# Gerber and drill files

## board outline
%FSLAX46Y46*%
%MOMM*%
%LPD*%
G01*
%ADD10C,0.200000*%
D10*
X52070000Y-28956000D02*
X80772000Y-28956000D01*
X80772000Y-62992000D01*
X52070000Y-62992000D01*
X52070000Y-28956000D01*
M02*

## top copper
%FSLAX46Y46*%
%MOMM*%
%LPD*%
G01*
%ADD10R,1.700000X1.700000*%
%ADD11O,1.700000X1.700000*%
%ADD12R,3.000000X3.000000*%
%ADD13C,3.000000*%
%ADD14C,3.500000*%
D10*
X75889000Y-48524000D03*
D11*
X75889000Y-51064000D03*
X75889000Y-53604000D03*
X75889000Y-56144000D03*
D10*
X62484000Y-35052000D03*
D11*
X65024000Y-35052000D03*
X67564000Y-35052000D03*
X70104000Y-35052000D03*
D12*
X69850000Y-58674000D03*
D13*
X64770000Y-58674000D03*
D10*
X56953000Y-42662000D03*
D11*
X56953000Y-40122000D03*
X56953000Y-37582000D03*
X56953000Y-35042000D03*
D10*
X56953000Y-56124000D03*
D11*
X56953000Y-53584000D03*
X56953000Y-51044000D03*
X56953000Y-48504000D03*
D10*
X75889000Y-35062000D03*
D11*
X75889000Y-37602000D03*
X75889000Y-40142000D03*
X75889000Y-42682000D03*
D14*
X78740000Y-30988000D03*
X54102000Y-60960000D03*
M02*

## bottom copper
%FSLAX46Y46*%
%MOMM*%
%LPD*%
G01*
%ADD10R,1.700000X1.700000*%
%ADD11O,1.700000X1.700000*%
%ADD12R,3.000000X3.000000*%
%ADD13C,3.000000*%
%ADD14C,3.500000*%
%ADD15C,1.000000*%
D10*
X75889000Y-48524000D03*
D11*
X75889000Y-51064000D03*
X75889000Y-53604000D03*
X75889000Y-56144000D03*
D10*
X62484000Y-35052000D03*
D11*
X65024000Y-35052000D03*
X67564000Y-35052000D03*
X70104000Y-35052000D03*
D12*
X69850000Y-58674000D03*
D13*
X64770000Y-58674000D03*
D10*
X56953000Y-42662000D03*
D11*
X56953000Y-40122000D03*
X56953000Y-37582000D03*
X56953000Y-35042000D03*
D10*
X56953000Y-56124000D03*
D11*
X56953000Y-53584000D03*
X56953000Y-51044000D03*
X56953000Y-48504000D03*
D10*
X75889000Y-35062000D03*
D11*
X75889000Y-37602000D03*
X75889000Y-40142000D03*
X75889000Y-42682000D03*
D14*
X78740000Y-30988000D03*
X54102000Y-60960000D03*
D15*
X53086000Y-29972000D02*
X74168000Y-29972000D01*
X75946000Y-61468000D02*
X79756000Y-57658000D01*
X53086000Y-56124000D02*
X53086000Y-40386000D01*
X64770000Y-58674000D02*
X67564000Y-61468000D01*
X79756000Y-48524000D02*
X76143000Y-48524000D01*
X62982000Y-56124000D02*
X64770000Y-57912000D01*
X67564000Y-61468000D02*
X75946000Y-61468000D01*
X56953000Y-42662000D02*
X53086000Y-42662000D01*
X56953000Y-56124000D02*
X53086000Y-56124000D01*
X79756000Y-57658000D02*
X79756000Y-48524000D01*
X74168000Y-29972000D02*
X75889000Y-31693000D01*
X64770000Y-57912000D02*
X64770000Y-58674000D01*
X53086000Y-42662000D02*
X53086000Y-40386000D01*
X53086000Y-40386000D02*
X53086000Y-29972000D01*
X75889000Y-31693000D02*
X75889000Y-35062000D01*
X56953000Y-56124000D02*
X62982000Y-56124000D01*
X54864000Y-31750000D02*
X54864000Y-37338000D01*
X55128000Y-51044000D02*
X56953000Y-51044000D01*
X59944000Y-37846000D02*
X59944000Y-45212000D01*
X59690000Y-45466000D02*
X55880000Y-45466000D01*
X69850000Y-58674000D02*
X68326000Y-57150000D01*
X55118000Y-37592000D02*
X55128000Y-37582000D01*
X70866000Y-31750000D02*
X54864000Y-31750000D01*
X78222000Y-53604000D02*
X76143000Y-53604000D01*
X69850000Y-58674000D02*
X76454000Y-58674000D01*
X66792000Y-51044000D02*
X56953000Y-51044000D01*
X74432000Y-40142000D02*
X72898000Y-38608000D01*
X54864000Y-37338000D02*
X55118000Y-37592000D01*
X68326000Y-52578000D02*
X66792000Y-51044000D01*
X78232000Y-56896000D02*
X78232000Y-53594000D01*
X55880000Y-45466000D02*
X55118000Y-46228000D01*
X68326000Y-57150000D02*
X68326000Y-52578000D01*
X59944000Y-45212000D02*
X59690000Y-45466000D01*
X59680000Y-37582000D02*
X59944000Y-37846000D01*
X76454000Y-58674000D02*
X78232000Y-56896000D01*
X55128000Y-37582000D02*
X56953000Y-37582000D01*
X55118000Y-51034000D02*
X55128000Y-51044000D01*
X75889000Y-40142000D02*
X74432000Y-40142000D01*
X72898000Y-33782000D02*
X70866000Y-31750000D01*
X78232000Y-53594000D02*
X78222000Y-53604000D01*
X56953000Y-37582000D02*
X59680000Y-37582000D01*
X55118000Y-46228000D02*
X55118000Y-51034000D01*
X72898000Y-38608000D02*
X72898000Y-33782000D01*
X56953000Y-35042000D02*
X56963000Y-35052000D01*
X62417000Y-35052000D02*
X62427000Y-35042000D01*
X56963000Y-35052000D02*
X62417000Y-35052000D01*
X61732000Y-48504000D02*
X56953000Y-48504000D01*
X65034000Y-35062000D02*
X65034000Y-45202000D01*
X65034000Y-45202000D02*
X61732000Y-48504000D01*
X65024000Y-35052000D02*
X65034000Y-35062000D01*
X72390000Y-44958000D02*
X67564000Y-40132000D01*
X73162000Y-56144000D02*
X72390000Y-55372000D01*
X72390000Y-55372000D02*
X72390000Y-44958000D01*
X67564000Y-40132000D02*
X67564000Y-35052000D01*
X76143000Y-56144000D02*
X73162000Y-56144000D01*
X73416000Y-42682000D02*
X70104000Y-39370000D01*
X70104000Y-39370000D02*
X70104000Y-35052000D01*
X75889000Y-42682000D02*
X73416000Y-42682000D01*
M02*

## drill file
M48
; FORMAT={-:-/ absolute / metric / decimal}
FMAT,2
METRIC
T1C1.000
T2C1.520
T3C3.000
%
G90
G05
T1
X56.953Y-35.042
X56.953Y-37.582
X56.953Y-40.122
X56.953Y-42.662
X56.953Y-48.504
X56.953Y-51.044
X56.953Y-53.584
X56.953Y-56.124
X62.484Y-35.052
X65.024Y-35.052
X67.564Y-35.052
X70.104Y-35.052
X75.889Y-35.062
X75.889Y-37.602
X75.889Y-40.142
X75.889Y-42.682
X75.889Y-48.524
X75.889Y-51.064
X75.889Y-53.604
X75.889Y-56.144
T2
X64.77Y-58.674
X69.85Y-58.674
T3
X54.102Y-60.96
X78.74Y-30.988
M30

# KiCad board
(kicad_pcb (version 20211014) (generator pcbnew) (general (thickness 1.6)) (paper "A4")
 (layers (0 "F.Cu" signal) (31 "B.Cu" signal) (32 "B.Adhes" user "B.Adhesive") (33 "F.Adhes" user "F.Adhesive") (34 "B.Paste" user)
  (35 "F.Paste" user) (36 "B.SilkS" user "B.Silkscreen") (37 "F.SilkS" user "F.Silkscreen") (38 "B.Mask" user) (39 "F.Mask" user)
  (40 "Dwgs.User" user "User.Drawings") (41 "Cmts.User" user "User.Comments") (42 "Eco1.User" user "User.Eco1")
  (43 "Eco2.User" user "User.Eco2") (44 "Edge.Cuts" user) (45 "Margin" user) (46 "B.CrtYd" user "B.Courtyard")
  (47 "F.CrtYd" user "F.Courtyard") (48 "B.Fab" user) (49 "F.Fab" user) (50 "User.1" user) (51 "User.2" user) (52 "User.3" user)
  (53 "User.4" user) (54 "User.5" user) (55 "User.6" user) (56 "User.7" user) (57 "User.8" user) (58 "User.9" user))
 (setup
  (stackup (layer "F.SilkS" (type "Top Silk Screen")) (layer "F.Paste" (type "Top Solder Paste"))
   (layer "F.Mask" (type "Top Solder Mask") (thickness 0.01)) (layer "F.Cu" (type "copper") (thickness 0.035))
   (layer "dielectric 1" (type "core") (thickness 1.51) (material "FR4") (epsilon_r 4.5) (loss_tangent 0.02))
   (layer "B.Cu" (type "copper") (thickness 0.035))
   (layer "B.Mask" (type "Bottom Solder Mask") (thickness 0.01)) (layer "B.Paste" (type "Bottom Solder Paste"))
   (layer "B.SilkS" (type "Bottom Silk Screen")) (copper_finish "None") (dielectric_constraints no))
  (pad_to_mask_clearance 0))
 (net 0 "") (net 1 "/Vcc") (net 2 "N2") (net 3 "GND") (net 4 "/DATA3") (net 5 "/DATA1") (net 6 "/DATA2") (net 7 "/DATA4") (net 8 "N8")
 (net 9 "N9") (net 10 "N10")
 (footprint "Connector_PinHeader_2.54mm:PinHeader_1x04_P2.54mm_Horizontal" (layer "F.Cu") (at 75.889 48.524)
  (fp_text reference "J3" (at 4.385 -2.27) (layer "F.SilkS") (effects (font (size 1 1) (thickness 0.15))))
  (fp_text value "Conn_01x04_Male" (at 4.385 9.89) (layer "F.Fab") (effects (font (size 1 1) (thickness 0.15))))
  (pad "1" thru_hole rect (at 0 0) (size 1.7 1.7) (drill 1) (layers *.Cu *.Mask) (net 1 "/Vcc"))
  (pad "2" thru_hole oval (at 0 2.54) (size 1.7 1.7) (drill 1) (layers *.Cu *.Mask) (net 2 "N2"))
  (pad "3" thru_hole oval (at 0 5.08) (size 1.7 1.7) (drill 1) (layers *.Cu *.Mask) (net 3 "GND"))
  (pad "4" thru_hole oval (at 0 7.62) (size 1.7 1.7) (drill 1) (layers *.Cu *.Mask) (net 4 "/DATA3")))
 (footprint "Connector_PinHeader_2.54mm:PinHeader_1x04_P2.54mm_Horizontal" (layer "F.Cu") (at 62.484 35.052 90)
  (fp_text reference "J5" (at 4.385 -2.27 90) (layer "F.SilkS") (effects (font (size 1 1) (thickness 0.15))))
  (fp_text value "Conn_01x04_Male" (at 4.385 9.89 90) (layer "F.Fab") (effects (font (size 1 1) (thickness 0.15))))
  (pad "1" thru_hole rect (at 0 0 90) (size 1.7 1.7) (drill 1) (layers *.Cu *.Mask) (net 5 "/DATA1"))
  (pad "2" thru_hole oval (at 0 2.54 90) (size 1.7 1.7) (drill 1) (layers *.Cu *.Mask) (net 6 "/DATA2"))
  (pad "3" thru_hole oval (at 0 5.08 90) (size 1.7 1.7) (drill 1) (layers *.Cu *.Mask) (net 4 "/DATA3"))
  (pad "4" thru_hole oval (at 0 7.62 90) (size 1.7 1.7) (drill 1) (layers *.Cu *.Mask) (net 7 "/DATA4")))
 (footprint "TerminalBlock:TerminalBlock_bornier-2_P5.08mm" (layer "F.Cu") (at 69.85 58.674 180)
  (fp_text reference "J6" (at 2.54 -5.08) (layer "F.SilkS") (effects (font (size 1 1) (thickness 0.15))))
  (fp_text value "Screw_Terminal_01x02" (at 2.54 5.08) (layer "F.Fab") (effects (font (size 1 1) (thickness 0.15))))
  (pad "1" thru_hole rect (at 0 0 180) (size 3 3) (drill 1.52) (layers *.Cu *.Mask) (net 3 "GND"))
  (pad "2" thru_hole circle (at 5.08 0 180) (size 3 3) (drill 1.52) (layers *.Cu *.Mask) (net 1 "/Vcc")))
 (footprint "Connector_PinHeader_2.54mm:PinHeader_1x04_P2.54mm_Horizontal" (layer "F.Cu") (at 56.953 42.662 180)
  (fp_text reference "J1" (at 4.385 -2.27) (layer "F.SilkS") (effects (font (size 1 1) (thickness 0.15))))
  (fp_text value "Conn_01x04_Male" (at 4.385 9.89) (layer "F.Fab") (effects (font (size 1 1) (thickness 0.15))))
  (pad "1" thru_hole rect (at 0 0 180) (size 1.7 1.7) (drill 1) (layers *.Cu *.Mask) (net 1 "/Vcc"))
  (pad "2" thru_hole oval (at 0 2.54 180) (size 1.7 1.7) (drill 1) (layers *.Cu *.Mask) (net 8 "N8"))
  (pad "3" thru_hole oval (at 0 5.08 180) (size 1.7 1.7) (drill 1) (layers *.Cu *.Mask) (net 3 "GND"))
  (pad "4" thru_hole oval (at 0 7.62 180) (size 1.7 1.7) (drill 1) (layers *.Cu *.Mask) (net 5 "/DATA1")))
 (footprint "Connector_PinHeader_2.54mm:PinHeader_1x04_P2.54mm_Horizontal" (layer "F.Cu") (at 56.953 56.124 180)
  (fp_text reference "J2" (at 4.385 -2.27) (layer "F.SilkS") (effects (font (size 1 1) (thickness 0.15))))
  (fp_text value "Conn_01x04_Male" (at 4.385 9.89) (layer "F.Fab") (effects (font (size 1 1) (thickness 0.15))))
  (pad "1" thru_hole rect (at 0 0 180) (size 1.7 1.7) (drill 1) (layers *.Cu *.Mask) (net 1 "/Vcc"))
  (pad "2" thru_hole oval (at 0 2.54 180) (size 1.7 1.7) (drill 1) (layers *.Cu *.Mask) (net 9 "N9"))
  (pad "3" thru_hole oval (at 0 5.08 180) (size 1.7 1.7) (drill 1) (layers *.Cu *.Mask) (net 3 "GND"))
  (pad "4" thru_hole oval (at 0 7.62 180) (size 1.7 1.7) (drill 1) (layers *.Cu *.Mask) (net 6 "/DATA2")))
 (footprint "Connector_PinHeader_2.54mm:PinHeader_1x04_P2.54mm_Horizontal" (layer "F.Cu") (at 75.889 35.062)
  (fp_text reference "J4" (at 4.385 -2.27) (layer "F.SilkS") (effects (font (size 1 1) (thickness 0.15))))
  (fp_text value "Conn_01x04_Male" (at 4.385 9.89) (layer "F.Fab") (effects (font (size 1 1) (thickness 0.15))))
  (pad "1" thru_hole rect (at 0 0) (size 1.7 1.7) (drill 1) (layers *.Cu *.Mask) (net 1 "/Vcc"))
  (pad "2" thru_hole oval (at 0 2.54) (size 1.7 1.7) (drill 1) (layers *.Cu *.Mask) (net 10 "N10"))
  (pad "3" thru_hole oval (at 0 5.08) (size 1.7 1.7) (drill 1) (layers *.Cu *.Mask) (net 3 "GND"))
  (pad "4" thru_hole oval (at 0 7.62) (size 1.7 1.7) (drill 1) (layers *.Cu *.Mask) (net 7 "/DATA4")))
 (gr_rect (start 52.07 28.956) (end 80.772 62.992) (layer "Edge.Cuts") (width 0.2) (fill none))
 (via (at 78.74 30.988) (size 3.5) (drill 3) (layers "F.Cu" "B.Cu") (free) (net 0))
 (via (at 54.102 60.96) (size 3.5) (drill 3) (layers "F.Cu" "B.Cu") (free) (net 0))
 (segment (start 53.086 29.972) (end 74.168 29.972) (width 1) (layer "B.Cu") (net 1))
 (segment (start 75.946 61.468) (end 79.756 57.658) (width 1) (layer "B.Cu") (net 1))
 (segment (start 53.086 56.124) (end 53.086 40.386) (width 1) (layer "B.Cu") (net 1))
 (segment (start 64.77 58.674) (end 67.564 61.468) (width 1) (layer "B.Cu") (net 1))
 (segment (start 79.756 48.524) (end 76.143 48.524) (width 1) (layer "B.Cu") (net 1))
 (segment (start 62.982 56.124) (end 64.77 57.912) (width 1) (layer "B.Cu") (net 1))
 (segment (start 67.564 61.468) (end 75.946 61.468) (width 1) (layer "B.Cu") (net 1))
 (segment (start 56.953 42.662) (end 53.086 42.662) (width 1) (layer "B.Cu") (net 1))
 (segment (start 56.953 56.124) (end 53.086 56.124) (width 1) (layer "B.Cu") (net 1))
 (segment (start 79.756 57.658) (end 79.756 48.524) (width 1) (layer "B.Cu") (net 1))
 (segment (start 74.168 29.972) (end 75.889 31.693) (width 1) (layer "B.Cu") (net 1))
 (segment (start 64.77 57.912) (end 64.77 58.674) (width 1) (layer "B.Cu") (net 1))
 (segment (start 53.086 42.662) (end 53.086 40.386) (width 1) (layer "B.Cu") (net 1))
 (segment (start 53.086 40.386) (end 53.086 29.972) (width 1) (layer "B.Cu") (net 1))
 (segment (start 75.889 31.693) (end 75.889 35.062) (width 1) (layer "B.Cu") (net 1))
 (segment (start 56.953 56.124) (end 62.982 56.124) (width 1) (layer "B.Cu") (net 1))
 (segment (start 54.864 31.75) (end 54.864 37.338) (width 1) (layer "B.Cu") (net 3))
 (segment (start 55.128 51.044) (end 56.953 51.044) (width 1) (layer "B.Cu") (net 3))
 (segment (start 59.944 37.846) (end 59.944 45.212) (width 1) (layer "B.Cu") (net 3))
 (segment (start 59.69 45.466) (end 55.88 45.466) (width 1) (layer "B.Cu") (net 3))
 (segment (start 69.85 58.674) (end 68.326 57.15) (width 1) (layer "B.Cu") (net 3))
 (segment (start 55.118 37.592) (end 55.128 37.582) (width 1) (layer "B.Cu") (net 3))
 (segment (start 70.866 31.75) (end 54.864 31.75) (width 1) (layer "B.Cu") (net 3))
 (segment (start 78.222 53.604) (end 76.143 53.604) (width 1) (layer "B.Cu") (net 3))
 (segment (start 69.85 58.674) (end 76.454 58.674) (width 1) (layer "B.Cu") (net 3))
 (segment (start 66.792 51.044) (end 56.953 51.044) (width 1) (layer "B.Cu") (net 3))
 (segment (start 74.432 40.142) (end 72.898 38.608) (width 1) (layer "B.Cu") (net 3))
 (segment (start 54.864 37.338) (end 55.118 37.592) (width 1) (layer "B.Cu") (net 3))
 (segment (start 68.326 52.578) (end 66.792 51.044) (width 1) (layer "B.Cu") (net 3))
 (segment (start 78.232 56.896) (end 78.232 53.594) (width 1) (layer "B.Cu") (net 3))
 (segment (start 55.88 45.466) (end 55.118 46.228) (width 1) (layer "B.Cu") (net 3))
 (segment (start 68.326 57.15) (end 68.326 52.578) (width 1) (layer "B.Cu") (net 3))
 (segment (start 59.944 45.212) (end 59.69 45.466) (width 1) (layer "B.Cu") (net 3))
 (segment (start 59.68 37.582) (end 59.944 37.846) (width 1) (layer "B.Cu") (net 3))
 (segment (start 76.454 58.674) (end 78.232 56.896) (width 1) (layer "B.Cu") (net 3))
 (segment (start 55.128 37.582) (end 56.953 37.582) (width 1) (layer "B.Cu") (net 3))
 (segment (start 55.118 51.034) (end 55.128 51.044) (width 1) (layer "B.Cu") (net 3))
 (segment (start 75.889 40.142) (end 74.432 40.142) (width 1) (layer "B.Cu") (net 3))
 (segment (start 72.898 33.782) (end 70.866 31.75) (width 1) (layer "B.Cu") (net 3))
 (segment (start 78.232 53.594) (end 78.222 53.604) (width 1) (layer "B.Cu") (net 3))
 (segment (start 56.953 37.582) (end 59.68 37.582) (width 1) (layer "B.Cu") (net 3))
 (segment (start 55.118 46.228) (end 55.118 51.034) (width 1) (layer "B.Cu") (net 3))
 (segment (start 72.898 38.608) (end 72.898 33.782) (width 1) (layer "B.Cu") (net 3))
 (segment (start 56.953 35.042) (end 56.963 35.052) (width 1) (layer "B.Cu") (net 5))
 (segment (start 62.417 35.052) (end 62.427 35.042) (width 1) (layer "B.Cu") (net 5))
 (segment (start 56.963 35.052) (end 62.417 35.052) (width 1) (layer "B.Cu") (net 5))
 (segment (start 61.732 48.504) (end 56.953 48.504) (width 1) (layer "B.Cu") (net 6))
 (segment (start 65.034 35.062) (end 65.034 45.202) (width 1) (layer "B.Cu") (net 6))
 (segment (start 65.034 45.202) (end 61.732 48.504) (width 1) (layer "B.Cu") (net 6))
 (segment (start 65.024 35.052) (end 65.034 35.062) (width 1) (layer "B.Cu") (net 6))
 (segment (start 72.39 44.958) (end 67.564 40.132) (width 1) (layer "B.Cu") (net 4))
 (segment (start 73.162 56.144) (end 72.39 55.372) (width 1) (layer "B.Cu") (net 4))
 (segment (start 72.39 55.372) (end 72.39 44.958) (width 1) (layer "B.Cu") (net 4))
 (segment (start 67.564 40.132) (end 67.564 35.052) (width 1) (layer "B.Cu") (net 4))
 (segment (start 76.143 56.144) (end 73.162 56.144) (width 1) (layer "B.Cu") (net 4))
 (segment (start 73.416 42.682) (end 70.104 39.37) (width 1) (layer "B.Cu") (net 7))
 (segment (start 70.104 39.37) (end 70.104 35.052) (width 1) (layer "B.Cu") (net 7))
 (segment (start 75.889 42.682) (end 73.416 42.682) (width 1) (layer "B.Cu") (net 7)))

